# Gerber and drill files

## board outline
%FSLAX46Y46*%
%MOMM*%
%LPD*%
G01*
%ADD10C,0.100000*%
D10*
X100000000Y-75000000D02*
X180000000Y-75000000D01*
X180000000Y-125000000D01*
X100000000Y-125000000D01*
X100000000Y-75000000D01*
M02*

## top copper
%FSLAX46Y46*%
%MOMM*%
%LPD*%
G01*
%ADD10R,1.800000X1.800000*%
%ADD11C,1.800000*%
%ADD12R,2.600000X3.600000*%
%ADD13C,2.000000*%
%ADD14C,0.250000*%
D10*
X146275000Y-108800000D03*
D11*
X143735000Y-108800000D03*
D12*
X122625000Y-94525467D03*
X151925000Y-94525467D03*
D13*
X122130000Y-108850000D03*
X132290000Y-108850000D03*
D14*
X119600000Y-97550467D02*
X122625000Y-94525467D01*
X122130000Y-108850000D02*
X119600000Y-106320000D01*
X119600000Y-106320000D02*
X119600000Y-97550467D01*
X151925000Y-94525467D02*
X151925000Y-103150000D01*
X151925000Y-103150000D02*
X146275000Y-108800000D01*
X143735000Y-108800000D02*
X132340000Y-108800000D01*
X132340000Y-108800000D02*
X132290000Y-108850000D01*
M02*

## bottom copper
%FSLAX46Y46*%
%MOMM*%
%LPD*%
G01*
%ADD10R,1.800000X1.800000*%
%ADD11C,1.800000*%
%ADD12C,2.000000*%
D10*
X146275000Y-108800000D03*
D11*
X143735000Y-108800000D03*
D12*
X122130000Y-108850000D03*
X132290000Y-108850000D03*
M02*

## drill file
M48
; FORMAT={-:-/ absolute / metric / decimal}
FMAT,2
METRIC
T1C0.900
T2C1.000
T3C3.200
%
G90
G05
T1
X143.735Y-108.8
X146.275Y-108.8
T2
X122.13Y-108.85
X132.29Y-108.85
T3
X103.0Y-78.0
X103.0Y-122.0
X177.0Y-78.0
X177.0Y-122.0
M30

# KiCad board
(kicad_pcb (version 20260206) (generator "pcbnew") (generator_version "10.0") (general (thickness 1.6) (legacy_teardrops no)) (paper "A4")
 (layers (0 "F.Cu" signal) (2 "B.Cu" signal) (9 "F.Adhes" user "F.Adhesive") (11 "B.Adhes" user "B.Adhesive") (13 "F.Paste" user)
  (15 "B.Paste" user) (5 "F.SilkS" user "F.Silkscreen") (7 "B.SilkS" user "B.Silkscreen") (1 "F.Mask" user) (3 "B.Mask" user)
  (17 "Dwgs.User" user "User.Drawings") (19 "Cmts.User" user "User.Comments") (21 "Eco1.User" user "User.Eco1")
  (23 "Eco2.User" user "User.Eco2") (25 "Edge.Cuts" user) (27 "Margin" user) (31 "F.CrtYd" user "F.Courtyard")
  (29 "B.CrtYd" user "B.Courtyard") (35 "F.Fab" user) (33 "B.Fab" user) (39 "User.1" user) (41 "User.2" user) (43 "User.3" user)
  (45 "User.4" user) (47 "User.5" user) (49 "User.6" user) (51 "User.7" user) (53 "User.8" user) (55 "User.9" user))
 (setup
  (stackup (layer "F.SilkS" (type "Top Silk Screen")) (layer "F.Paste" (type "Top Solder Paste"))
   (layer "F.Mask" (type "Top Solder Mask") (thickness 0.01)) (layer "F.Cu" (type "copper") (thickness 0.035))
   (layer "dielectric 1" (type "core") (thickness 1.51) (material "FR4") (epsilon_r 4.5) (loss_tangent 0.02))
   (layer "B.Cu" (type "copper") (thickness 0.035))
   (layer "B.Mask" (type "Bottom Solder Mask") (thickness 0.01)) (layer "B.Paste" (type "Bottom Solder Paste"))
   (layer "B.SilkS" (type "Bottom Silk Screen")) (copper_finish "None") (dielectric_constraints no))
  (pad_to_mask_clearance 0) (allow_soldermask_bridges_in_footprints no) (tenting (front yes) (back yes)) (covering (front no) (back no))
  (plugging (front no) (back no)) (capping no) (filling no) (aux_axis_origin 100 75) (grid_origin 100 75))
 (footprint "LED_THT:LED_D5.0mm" (layer "F.Cu") (at 146.275 108.8 180)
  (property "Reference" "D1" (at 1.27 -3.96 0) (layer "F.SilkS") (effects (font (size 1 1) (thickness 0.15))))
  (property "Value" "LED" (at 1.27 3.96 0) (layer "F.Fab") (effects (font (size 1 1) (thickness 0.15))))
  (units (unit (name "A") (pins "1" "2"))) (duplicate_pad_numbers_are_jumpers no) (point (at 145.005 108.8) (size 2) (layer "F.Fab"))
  (pad "1" thru_hole rect (at 0 0 180) (size 1.8 1.8) (drill 0.9) (layers "*.Cu" "*.Mask") (remove_unused_layers no) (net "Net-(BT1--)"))
  (pad "2" thru_hole circle (at 2.54 0 180) (size 1.8 1.8) (drill 0.9) (layers "*.Cu" "*.Mask") (remove_unused_layers no) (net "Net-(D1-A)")))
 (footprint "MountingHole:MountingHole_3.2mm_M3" (layer "F.Cu") (at 103 78)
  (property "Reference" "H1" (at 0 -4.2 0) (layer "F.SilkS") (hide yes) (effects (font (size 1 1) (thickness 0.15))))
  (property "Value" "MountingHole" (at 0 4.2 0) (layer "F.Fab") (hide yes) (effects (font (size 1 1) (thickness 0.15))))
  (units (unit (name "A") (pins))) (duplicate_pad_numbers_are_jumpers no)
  (pad "" np_thru_hole circle (at 0 0) (size 3.2 3.2) (drill 3.2) (layers "*.Cu" "*.Mask")))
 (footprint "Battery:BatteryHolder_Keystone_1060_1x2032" (layer "F.Cu") (at 137.275 94.525467)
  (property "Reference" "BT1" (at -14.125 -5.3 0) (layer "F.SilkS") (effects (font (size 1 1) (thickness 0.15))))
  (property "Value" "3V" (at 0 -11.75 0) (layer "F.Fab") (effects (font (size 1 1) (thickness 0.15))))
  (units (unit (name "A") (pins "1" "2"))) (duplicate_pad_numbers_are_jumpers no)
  (pad "1" smd rect (at -14.65 0 180) (size 2.6 3.6) (layers "F.Cu" "F.Mask" "F.Paste") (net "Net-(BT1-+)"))
  (pad "2" smd rect (at 14.65 0 180) (size 2.6 3.6) (layers "F.Cu" "F.Mask" "F.Paste") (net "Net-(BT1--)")))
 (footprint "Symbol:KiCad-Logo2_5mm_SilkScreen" (layer "F.Cu") (at 167 120)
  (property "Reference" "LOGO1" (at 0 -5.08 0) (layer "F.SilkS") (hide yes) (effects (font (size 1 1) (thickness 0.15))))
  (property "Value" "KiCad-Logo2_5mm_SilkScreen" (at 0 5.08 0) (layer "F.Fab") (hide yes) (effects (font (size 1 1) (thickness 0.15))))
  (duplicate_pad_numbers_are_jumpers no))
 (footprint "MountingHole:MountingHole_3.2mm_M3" (layer "F.Cu") (at 103 122)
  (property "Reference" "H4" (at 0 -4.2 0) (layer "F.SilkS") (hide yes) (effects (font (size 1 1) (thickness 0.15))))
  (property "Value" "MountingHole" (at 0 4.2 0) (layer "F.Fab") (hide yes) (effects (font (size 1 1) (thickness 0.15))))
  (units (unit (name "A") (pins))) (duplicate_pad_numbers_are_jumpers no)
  (pad "" np_thru_hole circle (at 0 0) (size 3.2 3.2) (drill 3.2) (layers "*.Cu" "*.Mask")))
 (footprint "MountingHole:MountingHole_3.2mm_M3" (layer "F.Cu") (at 177 122)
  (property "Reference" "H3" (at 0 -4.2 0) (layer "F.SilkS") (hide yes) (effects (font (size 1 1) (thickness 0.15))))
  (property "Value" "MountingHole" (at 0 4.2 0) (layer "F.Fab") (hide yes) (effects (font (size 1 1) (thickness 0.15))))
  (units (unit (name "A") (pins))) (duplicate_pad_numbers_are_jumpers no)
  (pad "" np_thru_hole circle (at 0 0) (size 3.2 3.2) (drill 3.2) (layers "*.Cu" "*.Mask")))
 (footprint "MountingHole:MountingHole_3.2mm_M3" (layer "F.Cu") (at 177 78)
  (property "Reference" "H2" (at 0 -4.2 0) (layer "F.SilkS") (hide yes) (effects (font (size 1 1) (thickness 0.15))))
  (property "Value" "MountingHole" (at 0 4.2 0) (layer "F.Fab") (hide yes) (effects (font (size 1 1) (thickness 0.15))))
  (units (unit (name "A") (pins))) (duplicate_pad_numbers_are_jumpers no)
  (pad "" np_thru_hole circle (at 0 0) (size 3.2 3.2) (drill 3.2) (layers "*.Cu" "*.Mask")))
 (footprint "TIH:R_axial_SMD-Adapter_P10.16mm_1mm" (layer "F.Cu") (at 122.13 108.85)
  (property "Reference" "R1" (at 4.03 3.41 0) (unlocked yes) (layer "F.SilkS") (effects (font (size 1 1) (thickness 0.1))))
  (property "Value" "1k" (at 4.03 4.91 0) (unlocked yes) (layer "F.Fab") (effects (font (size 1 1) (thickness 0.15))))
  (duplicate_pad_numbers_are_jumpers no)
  (pad "1" thru_hole circle (at 0 0) (size 2 2) (drill 1) (layers "*.Cu" "*.Mask") (remove_unused_layers no) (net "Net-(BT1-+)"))
  (pad "2" thru_hole circle (at 10.16 0) (size 2 2) (drill 1) (layers "*.Cu" "*.Mask") (remove_unused_layers no) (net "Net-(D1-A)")))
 (gr_rect (start 100 75) (end 180 125) (stroke (width 0.1) (type default)) (fill no) (layer "Edge.Cuts"))
 (segment (start 119.6 97.550467) (end 122.625 94.525467) (width 0.25) (layer "F.Cu") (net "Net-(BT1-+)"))
 (segment (start 122.13 108.85) (end 119.6 106.32) (width 0.25) (layer "F.Cu") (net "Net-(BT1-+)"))
 (segment (start 119.6 106.32) (end 119.6 97.550467) (width 0.25) (layer "F.Cu") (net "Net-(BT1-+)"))
 (segment (start 151.925 94.525467) (end 151.925 103.15) (width 0.25) (layer "F.Cu") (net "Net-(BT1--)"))
 (segment (start 151.925 103.15) (end 146.275 108.8) (width 0.25) (layer "F.Cu") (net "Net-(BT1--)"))
 (segment (start 143.735 108.8) (end 132.34 108.8) (width 0.25) (layer "F.Cu") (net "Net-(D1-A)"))
 (segment (start 132.34 108.8) (end 132.29 108.85) (width 0.25) (layer "F.Cu") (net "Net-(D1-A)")))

